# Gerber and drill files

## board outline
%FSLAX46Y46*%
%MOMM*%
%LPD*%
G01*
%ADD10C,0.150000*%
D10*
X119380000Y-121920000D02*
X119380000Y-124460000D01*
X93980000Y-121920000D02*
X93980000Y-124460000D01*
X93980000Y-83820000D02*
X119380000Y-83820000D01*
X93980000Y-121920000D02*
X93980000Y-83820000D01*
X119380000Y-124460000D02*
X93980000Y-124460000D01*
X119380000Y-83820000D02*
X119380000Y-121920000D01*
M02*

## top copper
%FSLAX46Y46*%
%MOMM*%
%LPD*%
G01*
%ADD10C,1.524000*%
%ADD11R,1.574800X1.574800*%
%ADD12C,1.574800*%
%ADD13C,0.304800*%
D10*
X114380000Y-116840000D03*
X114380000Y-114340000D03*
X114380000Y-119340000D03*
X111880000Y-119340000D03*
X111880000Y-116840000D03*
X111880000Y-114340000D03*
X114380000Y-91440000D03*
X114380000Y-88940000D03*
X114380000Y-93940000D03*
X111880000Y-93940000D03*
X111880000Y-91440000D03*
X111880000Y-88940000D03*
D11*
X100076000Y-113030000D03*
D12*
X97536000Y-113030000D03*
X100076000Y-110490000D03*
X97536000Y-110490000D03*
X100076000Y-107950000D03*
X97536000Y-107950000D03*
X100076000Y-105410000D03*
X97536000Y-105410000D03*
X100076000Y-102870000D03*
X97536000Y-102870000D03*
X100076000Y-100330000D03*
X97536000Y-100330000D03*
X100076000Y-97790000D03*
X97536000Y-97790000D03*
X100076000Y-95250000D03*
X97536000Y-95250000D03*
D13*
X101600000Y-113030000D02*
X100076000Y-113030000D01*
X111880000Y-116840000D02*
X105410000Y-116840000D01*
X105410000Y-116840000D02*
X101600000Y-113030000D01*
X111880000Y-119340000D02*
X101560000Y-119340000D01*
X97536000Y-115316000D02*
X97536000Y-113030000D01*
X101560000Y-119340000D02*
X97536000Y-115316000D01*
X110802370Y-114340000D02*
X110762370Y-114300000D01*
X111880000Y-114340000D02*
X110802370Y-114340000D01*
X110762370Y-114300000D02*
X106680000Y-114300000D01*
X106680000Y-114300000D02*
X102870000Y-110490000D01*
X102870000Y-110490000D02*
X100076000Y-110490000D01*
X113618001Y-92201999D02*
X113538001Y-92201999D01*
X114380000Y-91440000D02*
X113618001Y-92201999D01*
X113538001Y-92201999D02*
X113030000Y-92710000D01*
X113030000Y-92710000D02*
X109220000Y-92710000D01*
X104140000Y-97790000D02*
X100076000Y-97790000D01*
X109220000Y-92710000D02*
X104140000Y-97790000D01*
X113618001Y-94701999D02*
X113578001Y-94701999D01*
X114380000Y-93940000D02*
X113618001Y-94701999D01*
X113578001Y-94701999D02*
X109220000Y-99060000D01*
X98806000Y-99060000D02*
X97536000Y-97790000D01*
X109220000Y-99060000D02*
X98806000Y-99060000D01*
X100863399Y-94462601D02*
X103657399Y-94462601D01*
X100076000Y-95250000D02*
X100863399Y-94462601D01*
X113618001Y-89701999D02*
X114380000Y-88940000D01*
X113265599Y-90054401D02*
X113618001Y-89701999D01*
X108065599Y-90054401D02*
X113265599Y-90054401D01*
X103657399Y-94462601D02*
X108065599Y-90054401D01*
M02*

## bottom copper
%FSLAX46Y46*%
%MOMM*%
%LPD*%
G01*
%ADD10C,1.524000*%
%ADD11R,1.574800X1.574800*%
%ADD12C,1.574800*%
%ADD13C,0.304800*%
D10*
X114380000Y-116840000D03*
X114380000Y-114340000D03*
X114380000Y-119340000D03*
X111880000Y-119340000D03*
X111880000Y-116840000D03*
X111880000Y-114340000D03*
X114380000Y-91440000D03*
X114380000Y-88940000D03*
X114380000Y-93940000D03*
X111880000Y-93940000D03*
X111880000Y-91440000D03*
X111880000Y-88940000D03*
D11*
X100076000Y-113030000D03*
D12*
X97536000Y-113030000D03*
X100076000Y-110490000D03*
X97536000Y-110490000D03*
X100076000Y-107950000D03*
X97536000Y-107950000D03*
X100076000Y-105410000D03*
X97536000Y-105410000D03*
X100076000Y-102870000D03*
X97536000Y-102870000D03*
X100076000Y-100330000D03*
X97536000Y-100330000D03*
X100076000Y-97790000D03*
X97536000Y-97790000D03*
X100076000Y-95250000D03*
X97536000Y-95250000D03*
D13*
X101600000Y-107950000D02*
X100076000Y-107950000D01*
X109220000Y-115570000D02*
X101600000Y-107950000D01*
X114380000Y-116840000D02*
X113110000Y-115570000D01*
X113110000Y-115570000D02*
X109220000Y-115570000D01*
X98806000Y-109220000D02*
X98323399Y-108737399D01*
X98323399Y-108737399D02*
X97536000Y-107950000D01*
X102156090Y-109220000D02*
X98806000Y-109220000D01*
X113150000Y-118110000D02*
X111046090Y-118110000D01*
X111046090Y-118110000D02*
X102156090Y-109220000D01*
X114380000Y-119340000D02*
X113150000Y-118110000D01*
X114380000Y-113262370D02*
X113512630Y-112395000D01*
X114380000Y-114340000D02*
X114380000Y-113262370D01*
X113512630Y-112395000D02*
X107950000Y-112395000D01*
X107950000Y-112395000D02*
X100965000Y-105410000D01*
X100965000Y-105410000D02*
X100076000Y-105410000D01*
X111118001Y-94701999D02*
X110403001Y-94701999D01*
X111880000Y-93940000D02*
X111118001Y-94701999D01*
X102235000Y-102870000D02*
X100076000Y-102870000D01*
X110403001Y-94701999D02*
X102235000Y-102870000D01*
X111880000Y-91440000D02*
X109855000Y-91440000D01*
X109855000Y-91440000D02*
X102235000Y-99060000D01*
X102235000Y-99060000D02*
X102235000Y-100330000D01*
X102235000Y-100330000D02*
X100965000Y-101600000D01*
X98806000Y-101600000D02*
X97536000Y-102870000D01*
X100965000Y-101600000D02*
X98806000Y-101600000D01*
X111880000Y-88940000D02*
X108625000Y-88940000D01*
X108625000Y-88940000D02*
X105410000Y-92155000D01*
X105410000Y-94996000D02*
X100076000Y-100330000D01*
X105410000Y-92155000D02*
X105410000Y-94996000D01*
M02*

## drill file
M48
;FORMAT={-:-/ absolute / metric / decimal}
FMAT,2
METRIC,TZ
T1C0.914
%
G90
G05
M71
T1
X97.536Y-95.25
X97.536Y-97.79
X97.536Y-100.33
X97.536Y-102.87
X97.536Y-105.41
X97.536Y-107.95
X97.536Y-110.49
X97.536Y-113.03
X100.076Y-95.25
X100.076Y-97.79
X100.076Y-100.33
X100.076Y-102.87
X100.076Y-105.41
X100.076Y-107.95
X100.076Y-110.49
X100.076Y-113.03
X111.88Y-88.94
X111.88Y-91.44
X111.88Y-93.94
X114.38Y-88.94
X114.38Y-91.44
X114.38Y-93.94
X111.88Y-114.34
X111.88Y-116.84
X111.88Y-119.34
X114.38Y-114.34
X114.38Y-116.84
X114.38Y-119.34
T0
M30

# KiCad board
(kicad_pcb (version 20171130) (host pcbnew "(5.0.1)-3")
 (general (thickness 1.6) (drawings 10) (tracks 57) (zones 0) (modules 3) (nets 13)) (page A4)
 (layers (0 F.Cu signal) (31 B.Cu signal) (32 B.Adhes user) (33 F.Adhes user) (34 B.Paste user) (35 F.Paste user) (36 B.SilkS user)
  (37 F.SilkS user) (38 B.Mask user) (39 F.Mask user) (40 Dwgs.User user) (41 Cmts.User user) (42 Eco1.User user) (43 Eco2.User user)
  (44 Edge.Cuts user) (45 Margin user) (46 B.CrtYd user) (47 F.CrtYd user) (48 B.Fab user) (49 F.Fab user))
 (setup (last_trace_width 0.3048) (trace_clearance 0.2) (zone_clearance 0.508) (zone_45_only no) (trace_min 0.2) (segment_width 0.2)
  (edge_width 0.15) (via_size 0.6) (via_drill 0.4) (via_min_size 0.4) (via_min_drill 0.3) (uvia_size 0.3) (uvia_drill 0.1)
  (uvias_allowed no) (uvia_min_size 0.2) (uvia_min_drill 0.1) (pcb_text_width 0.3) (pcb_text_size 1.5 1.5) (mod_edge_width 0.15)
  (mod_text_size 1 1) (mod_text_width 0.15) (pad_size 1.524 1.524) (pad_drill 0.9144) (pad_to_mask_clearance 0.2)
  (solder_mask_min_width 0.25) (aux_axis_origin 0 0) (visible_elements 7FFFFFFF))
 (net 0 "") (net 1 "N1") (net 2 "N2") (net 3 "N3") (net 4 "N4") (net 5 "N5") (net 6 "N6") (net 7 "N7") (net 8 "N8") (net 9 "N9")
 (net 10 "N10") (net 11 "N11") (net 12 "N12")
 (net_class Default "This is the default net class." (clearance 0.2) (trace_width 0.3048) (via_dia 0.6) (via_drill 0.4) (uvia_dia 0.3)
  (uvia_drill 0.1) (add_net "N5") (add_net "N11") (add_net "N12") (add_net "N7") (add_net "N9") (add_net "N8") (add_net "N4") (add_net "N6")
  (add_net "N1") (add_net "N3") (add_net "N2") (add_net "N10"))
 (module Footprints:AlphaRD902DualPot (layer F.Cu) (at 119.38 116.84)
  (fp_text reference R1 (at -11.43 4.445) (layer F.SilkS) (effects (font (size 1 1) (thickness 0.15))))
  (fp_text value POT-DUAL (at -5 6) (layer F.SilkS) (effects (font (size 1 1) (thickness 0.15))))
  (pad 2 thru_hole circle (at -5 0) (size 1.524 1.524) (drill 0.9144) (layers *.Cu *.Mask F.SilkS) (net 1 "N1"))
  (pad 3 thru_hole circle (at -5 -2.5) (size 1.524 1.524) (drill 0.9144) (layers *.Cu *.Mask F.SilkS) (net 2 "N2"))
  (pad 1 thru_hole circle (at -5 2.5) (size 1.524 1.524) (drill 0.9144) (layers *.Cu *.Mask F.SilkS) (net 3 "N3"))
  (pad 4 thru_hole circle (at -7.5 2.5) (size 1.524 1.524) (drill 0.9144) (layers *.Cu *.Mask F.SilkS) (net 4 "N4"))
  (pad 5 thru_hole circle (at -7.5 0) (size 1.524 1.524) (drill 0.9144) (layers *.Cu *.Mask F.SilkS) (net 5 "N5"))
  (pad 6 thru_hole circle (at -7.5 -2.5) (size 1.524 1.524) (drill 0.9144) (layers *.Cu *.Mask F.SilkS) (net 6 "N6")))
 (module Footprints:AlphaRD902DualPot (layer F.Cu) (at 119.38 91.44)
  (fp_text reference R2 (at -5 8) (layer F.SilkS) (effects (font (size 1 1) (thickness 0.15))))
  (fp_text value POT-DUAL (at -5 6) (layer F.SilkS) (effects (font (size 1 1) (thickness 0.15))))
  (pad 2 thru_hole circle (at -5 0) (size 1.524 1.524) (drill 0.9144) (layers *.Cu *.Mask F.SilkS) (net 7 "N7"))
  (pad 3 thru_hole circle (at -5 -2.5) (size 1.524 1.524) (drill 0.9144) (layers *.Cu *.Mask F.SilkS) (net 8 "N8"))
  (pad 1 thru_hole circle (at -5 2.5) (size 1.524 1.524) (drill 0.9144) (layers *.Cu *.Mask F.SilkS) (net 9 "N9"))
  (pad 4 thru_hole circle (at -7.5 2.5) (size 1.524 1.524) (drill 0.9144) (layers *.Cu *.Mask F.SilkS) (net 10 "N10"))
  (pad 5 thru_hole circle (at -7.5 0) (size 1.524 1.524) (drill 0.9144) (layers *.Cu *.Mask F.SilkS) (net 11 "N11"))
  (pad 6 thru_hole circle (at -7.5 -2.5) (size 1.524 1.524) (drill 0.9144) (layers *.Cu *.Mask F.SilkS) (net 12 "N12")))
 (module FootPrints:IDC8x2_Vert (layer F.Cu) (at 98.806 104.14 270)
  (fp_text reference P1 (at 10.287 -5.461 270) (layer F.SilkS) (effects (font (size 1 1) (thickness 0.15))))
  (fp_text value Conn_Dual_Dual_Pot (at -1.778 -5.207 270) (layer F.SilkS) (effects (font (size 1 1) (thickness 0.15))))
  (pad 1 thru_hole rect (at 8.89 -1.27 270) (size 1.5748 1.5748) (drill 0.9144) (layers *.Cu *.Mask F.SilkS) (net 5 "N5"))
  (pad 2 thru_hole circle (at 8.89 1.27 270) (size 1.5748 1.5748) (drill 0.9144) (layers *.Cu *.Mask F.SilkS) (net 4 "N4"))
  (pad 3 thru_hole circle (at 6.35 -1.27 270) (size 1.5748 1.5748) (drill 0.9144) (layers *.Cu *.Mask F.SilkS) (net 6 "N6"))
  (pad 4 thru_hole circle (at 6.35 1.27 270) (size 1.5748 1.5748) (drill 0.9144) (layers *.Cu *.Mask F.SilkS))
  (pad 5 thru_hole circle (at 3.81 -1.27 270) (size 1.5748 1.5748) (drill 0.9144) (layers *.Cu *.Mask F.SilkS) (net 1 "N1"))
  (pad 6 thru_hole circle (at 3.81 1.27 270) (size 1.5748 1.5748) (drill 0.9144) (layers *.Cu *.Mask F.SilkS) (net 3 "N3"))
  (pad 7 thru_hole circle (at 1.27 -1.27 270) (size 1.5748 1.5748) (drill 0.9144) (layers *.Cu *.Mask F.SilkS) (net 2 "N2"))
  (pad 8 thru_hole circle (at 1.27 1.27 270) (size 1.5748 1.5748) (drill 0.9144) (layers *.Cu *.Mask F.SilkS))
  (pad 9 thru_hole circle (at -1.27 -1.27 270) (size 1.5748 1.5748) (drill 0.9144) (layers *.Cu *.Mask F.SilkS) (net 10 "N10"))
  (pad 10 thru_hole circle (at -1.27 1.27 270) (size 1.5748 1.5748) (drill 0.9144) (layers *.Cu *.Mask F.SilkS) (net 11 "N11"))
  (pad 11 thru_hole circle (at -3.81 -1.27 270) (size 1.5748 1.5748) (drill 0.9144) (layers *.Cu *.Mask F.SilkS) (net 12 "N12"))
  (pad 12 thru_hole circle (at -3.81 1.27 270) (size 1.5748 1.5748) (drill 0.9144) (layers *.Cu *.Mask F.SilkS))
  (pad 13 thru_hole circle (at -6.35 -1.27 270) (size 1.5748 1.5748) (drill 0.9144) (layers *.Cu *.Mask F.SilkS) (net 7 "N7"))
  (pad 14 thru_hole circle (at -6.35 1.27 270) (size 1.5748 1.5748) (drill 0.9144) (layers *.Cu *.Mask F.SilkS) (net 9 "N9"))
  (pad 15 thru_hole circle (at -8.89 -1.27 270) (size 1.5748 1.5748) (drill 0.9144) (layers *.Cu *.Mask F.SilkS) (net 8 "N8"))
  (pad 16 thru_hole circle (at -8.89 1.27 270) (size 1.5748 1.5748) (drill 0.9144) (layers *.Cu *.Mask F.SilkS)))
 (gr_line (start 119.38 121.92) (end 119.38 124.46) (angle 90) (layer Edge.Cuts) (width 0.15))
 (gr_line (start 93.98 121.92) (end 93.98 124.46) (angle 90) (layer Edge.Cuts) (width 0.15))
 (gr_line (start 93.98 83.82) (end 119.38 83.82) (angle 90) (layer Edge.Cuts) (width 0.15))
 (gr_line (start 93.98 121.92) (end 93.98 83.82) (angle 90) (layer Edge.Cuts) (width 0.15))
 (gr_line (start 119.38 124.46) (end 93.98 124.46) (angle 90) (layer Edge.Cuts) (width 0.15))
 (gr_line (start 119.38 83.82) (end 119.38 121.92) (angle 90) (layer Edge.Cuts) (width 0.15))
 (segment (start 101.6 113.03) (end 100.076 113.03) (width 0.3048) (layer F.Cu) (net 5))
 (segment (start 111.88 116.84) (end 105.41 116.84) (width 0.3048) (layer F.Cu) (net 5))
 (segment (start 105.41 116.84) (end 101.6 113.03) (width 0.3048) (layer F.Cu) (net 5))
 (segment (start 111.88 119.34) (end 101.56 119.34) (width 0.3048) (layer F.Cu) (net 4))
 (segment (start 97.536 115.316) (end 97.536 113.03) (width 0.3048) (layer F.Cu) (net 4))
 (segment (start 101.56 119.34) (end 97.536 115.316) (width 0.3048) (layer F.Cu) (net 4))
 (segment (start 110.80237 114.34) (end 110.76237 114.3) (width 0.3048) (layer F.Cu) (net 6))
 (segment (start 111.88 114.34) (end 110.80237 114.34) (width 0.3048) (layer F.Cu) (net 6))
 (segment (start 110.76237 114.3) (end 106.68 114.3) (width 0.3048) (layer F.Cu) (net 6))
 (segment (start 106.68 114.3) (end 102.87 110.49) (width 0.3048) (layer F.Cu) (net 6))
 (segment (start 102.87 110.49) (end 100.076 110.49) (width 0.3048) (layer F.Cu) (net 6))
 (segment (start 101.6 107.95) (end 100.076 107.95) (width 0.3048) (layer B.Cu) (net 1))
 (segment (start 109.22 115.57) (end 101.6 107.95) (width 0.3048) (layer B.Cu) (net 1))
 (segment (start 114.38 116.84) (end 113.11 115.57) (width 0.3048) (layer B.Cu) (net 1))
 (segment (start 113.11 115.57) (end 109.22 115.57) (width 0.3048) (layer B.Cu) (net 1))
 (segment (start 98.806 109.22) (end 98.323399 108.737399) (width 0.3048) (layer B.Cu) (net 3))
 (segment (start 98.323399 108.737399) (end 97.536 107.95) (width 0.3048) (layer B.Cu) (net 3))
 (segment (start 102.15609 109.22) (end 98.806 109.22) (width 0.3048) (layer B.Cu) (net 3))
 (segment (start 113.15 118.11) (end 111.04609 118.11) (width 0.3048) (layer B.Cu) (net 3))
 (segment (start 111.04609 118.11) (end 102.15609 109.22) (width 0.3048) (layer B.Cu) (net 3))
 (segment (start 114.38 119.34) (end 113.15 118.11) (width 0.3048) (layer B.Cu) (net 3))
 (segment (start 114.38 113.26237) (end 113.51263 112.395) (width 0.3048) (layer B.Cu) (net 2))
 (segment (start 114.38 114.34) (end 114.38 113.26237) (width 0.3048) (layer B.Cu) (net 2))
 (segment (start 113.51263 112.395) (end 107.95 112.395) (width 0.3048) (layer B.Cu) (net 2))
 (segment (start 107.95 112.395) (end 100.965 105.41) (width 0.3048) (layer B.Cu) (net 2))
 (segment (start 100.965 105.41) (end 100.076 105.41) (width 0.3048) (layer B.Cu) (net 2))
 (segment (start 111.118001 94.701999) (end 110.403001 94.701999) (width 0.3048) (layer B.Cu) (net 10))
 (segment (start 111.88 93.94) (end 111.118001 94.701999) (width 0.3048) (layer B.Cu) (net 10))
 (segment (start 102.235 102.87) (end 100.076 102.87) (width 0.3048) (layer B.Cu) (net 10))
 (segment (start 110.403001 94.701999) (end 102.235 102.87) (width 0.3048) (layer B.Cu) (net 10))
 (segment (start 111.88 91.44) (end 109.855 91.44) (width 0.3048) (layer B.Cu) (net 11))
 (segment (start 109.855 91.44) (end 102.235 99.06) (width 0.3048) (layer B.Cu) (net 11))
 (segment (start 102.235 99.06) (end 102.235 100.33) (width 0.3048) (layer B.Cu) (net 11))
 (segment (start 102.235 100.33) (end 100.965 101.6) (width 0.3048) (layer B.Cu) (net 11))
 (segment (start 98.806 101.6) (end 97.536 102.87) (width 0.3048) (layer B.Cu) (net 11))
 (segment (start 100.965 101.6) (end 98.806 101.6) (width 0.3048) (layer B.Cu) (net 11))
 (segment (start 111.88 88.94) (end 108.625 88.94) (width 0.3048) (layer B.Cu) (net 12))
 (segment (start 108.625 88.94) (end 105.41 92.155) (width 0.3048) (layer B.Cu) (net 12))
 (segment (start 105.41 94.996) (end 100.076 100.33) (width 0.3048) (layer B.Cu) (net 12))
 (segment (start 105.41 92.155) (end 105.41 94.996) (width 0.3048) (layer B.Cu) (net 12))
 (segment (start 113.618001 92.201999) (end 113.538001 92.201999) (width 0.3048) (layer F.Cu) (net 7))
 (segment (start 114.38 91.44) (end 113.618001 92.201999) (width 0.3048) (layer F.Cu) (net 7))
 (segment (start 113.538001 92.201999) (end 113.03 92.71) (width 0.3048) (layer F.Cu) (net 7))
 (segment (start 113.03 92.71) (end 109.22 92.71) (width 0.3048) (layer F.Cu) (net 7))
 (segment (start 104.14 97.79) (end 100.076 97.79) (width 0.3048) (layer F.Cu) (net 7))
 (segment (start 109.22 92.71) (end 104.14 97.79) (width 0.3048) (layer F.Cu) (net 7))
 (segment (start 113.618001 94.701999) (end 113.578001 94.701999) (width 0.3048) (layer F.Cu) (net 9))
 (segment (start 114.38 93.94) (end 113.618001 94.701999) (width 0.3048) (layer F.Cu) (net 9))
 (segment (start 113.578001 94.701999) (end 109.22 99.06) (width 0.3048) (layer F.Cu) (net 9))
 (segment (start 98.806 99.06) (end 97.536 97.79) (width 0.3048) (layer F.Cu) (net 9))
 (segment (start 109.22 99.06) (end 98.806 99.06) (width 0.3048) (layer F.Cu) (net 9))
 (segment (start 100.863399 94.462601) (end 103.657399 94.462601) (width 0.3048) (layer F.Cu) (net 8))
 (segment (start 100.076 95.25) (end 100.863399 94.462601) (width 0.3048) (layer F.Cu) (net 8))
 (segment (start 113.618001 89.701999) (end 114.38 88.94) (width 0.3048) (layer F.Cu) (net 8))
 (segment (start 113.265599 90.054401) (end 113.618001 89.701999) (width 0.3048) (layer F.Cu) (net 8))
 (segment (start 108.065599 90.054401) (end 113.265599 90.054401) (width 0.3048) (layer F.Cu) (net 8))
 (segment (start 103.657399 94.462601) (end 108.065599 90.054401) (width 0.3048) (layer F.Cu) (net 8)))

